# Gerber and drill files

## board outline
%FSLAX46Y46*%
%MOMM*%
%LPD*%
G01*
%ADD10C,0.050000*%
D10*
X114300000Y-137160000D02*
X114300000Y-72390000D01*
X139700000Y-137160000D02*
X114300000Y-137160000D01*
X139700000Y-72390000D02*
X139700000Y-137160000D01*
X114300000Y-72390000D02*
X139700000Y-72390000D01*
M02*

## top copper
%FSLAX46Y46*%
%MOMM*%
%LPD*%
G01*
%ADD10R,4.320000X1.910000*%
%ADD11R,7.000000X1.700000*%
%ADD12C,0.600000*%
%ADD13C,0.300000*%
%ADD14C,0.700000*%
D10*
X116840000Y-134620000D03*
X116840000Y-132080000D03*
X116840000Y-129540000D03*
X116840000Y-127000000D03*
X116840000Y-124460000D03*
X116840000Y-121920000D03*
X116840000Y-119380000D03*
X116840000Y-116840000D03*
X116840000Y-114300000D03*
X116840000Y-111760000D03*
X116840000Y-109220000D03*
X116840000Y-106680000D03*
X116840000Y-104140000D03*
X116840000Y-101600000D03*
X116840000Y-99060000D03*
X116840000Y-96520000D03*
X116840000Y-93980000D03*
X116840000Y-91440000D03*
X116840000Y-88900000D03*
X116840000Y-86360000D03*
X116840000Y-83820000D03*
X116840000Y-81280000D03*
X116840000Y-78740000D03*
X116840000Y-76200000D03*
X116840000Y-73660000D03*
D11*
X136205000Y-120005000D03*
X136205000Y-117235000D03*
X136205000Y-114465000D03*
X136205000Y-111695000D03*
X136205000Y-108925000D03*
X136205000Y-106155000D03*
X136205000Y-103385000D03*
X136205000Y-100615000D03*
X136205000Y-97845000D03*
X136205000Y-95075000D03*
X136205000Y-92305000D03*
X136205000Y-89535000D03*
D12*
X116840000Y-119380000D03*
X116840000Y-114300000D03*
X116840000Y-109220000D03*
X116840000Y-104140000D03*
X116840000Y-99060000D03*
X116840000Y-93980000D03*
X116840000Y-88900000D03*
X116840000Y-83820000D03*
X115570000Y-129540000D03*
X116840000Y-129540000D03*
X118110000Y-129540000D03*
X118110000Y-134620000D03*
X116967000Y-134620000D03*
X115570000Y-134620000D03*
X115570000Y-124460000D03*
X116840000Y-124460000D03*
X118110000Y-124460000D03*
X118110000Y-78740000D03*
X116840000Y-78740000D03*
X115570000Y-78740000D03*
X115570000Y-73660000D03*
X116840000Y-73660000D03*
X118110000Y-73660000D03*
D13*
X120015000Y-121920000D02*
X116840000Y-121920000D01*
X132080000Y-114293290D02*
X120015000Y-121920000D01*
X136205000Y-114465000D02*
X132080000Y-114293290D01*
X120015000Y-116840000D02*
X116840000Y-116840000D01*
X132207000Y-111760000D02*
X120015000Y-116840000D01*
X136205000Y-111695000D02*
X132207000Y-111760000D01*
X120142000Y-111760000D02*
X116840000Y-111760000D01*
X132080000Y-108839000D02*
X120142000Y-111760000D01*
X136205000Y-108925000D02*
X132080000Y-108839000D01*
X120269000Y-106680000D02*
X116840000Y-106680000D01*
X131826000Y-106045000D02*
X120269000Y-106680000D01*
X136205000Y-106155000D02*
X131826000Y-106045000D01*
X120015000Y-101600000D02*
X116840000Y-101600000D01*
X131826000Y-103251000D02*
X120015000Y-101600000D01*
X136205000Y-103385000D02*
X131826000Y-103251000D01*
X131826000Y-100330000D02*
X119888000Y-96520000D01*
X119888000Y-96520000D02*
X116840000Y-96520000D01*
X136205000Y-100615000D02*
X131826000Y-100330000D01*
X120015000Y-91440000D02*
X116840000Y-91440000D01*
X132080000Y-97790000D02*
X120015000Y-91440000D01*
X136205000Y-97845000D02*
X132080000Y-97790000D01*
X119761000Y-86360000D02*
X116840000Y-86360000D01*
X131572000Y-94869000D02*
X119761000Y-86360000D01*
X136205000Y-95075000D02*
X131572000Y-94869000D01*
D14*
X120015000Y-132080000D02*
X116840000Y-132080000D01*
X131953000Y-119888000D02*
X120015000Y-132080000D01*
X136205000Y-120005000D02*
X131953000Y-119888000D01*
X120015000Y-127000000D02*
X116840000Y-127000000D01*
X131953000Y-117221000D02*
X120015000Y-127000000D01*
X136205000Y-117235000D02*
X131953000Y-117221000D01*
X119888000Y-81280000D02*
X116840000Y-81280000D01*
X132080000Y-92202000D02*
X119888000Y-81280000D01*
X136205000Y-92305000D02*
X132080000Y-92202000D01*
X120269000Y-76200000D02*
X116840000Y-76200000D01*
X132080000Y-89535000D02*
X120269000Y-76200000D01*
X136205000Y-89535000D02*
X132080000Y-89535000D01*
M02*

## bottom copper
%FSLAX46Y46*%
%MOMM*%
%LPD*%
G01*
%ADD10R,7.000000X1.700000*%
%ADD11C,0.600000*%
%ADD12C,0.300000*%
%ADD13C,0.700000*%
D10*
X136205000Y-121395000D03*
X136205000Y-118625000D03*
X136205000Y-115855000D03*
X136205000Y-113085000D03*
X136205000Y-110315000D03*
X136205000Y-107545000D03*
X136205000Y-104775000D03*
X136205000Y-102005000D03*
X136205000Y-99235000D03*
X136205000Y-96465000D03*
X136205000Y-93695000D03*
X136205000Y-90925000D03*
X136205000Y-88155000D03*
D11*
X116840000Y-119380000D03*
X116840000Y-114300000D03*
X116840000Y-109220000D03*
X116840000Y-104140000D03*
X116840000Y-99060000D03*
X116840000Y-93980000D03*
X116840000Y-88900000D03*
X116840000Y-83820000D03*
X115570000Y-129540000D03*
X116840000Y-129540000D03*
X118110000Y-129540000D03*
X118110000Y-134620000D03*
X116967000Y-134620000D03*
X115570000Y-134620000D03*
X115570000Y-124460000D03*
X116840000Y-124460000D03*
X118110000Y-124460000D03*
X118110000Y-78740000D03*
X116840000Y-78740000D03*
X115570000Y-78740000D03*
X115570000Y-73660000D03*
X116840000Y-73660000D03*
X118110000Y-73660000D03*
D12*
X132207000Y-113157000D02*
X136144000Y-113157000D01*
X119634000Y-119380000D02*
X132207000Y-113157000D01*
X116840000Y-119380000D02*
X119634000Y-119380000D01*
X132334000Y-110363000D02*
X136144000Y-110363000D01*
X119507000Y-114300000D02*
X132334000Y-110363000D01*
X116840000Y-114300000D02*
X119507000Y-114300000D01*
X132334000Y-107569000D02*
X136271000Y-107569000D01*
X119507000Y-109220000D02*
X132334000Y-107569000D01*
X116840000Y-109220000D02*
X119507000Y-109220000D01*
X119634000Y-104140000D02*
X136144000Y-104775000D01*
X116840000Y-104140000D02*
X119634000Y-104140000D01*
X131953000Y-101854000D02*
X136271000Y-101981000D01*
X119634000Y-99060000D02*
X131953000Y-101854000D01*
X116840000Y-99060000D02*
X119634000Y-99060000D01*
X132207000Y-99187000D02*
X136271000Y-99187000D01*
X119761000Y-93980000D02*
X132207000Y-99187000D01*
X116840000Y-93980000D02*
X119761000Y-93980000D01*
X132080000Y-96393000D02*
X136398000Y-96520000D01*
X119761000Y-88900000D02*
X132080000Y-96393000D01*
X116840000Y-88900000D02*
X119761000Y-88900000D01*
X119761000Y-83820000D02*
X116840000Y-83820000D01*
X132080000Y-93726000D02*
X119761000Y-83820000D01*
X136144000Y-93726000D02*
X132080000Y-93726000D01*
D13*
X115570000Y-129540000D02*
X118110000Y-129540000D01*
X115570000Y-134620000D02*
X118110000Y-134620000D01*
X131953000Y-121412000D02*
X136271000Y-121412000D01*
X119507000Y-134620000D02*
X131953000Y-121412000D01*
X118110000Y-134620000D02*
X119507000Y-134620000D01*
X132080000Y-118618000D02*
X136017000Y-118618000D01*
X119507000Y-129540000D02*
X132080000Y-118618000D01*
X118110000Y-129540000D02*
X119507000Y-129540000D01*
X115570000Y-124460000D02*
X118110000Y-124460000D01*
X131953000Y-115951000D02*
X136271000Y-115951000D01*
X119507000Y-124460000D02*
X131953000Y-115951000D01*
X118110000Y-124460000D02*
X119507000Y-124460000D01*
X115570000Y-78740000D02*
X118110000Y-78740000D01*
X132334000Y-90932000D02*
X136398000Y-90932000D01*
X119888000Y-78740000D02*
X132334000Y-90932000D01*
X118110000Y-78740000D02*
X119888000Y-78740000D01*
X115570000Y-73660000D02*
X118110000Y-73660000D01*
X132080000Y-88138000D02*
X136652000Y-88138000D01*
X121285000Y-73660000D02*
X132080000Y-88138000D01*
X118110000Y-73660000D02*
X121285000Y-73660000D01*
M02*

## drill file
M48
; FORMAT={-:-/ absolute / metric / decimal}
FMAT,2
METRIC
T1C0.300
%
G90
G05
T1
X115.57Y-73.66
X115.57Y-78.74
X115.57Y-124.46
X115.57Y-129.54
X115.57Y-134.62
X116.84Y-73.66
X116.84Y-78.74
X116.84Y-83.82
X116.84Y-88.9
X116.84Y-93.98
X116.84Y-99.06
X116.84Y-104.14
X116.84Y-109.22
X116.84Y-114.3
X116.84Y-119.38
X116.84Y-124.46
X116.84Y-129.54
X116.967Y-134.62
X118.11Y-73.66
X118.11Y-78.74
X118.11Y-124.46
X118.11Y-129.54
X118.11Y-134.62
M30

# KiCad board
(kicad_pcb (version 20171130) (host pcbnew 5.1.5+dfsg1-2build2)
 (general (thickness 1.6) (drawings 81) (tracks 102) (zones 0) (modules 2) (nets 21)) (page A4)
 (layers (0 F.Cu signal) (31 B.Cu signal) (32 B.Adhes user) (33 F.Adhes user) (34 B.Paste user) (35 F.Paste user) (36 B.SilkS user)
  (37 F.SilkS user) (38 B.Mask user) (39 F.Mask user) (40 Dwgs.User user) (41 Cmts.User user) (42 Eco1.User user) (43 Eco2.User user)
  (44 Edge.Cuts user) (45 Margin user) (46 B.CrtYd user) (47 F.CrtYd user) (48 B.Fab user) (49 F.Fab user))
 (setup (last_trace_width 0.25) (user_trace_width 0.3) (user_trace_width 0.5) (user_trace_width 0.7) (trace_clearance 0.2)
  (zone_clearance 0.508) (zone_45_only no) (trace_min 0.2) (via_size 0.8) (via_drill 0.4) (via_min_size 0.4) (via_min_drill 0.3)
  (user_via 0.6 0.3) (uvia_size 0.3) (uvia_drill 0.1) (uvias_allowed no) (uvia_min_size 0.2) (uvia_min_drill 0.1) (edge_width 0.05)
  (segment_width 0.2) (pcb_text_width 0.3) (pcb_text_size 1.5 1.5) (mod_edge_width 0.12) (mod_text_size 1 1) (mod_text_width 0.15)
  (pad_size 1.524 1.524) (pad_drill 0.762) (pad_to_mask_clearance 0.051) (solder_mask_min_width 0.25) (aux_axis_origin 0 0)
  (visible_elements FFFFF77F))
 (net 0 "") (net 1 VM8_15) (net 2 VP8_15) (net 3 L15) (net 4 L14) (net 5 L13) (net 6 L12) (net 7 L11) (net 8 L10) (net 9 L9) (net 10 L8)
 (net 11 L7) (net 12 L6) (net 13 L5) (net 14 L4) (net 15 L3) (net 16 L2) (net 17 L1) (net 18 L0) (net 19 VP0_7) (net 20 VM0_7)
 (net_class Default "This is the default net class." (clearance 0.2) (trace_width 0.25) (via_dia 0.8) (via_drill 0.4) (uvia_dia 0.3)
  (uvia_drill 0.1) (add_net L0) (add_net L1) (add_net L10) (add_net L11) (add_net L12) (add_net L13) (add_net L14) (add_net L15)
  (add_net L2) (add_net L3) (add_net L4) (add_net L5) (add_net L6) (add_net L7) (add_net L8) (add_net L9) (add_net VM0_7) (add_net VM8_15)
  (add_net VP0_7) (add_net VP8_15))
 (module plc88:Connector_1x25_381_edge (layer F.Cu) (at 111.76 71.12)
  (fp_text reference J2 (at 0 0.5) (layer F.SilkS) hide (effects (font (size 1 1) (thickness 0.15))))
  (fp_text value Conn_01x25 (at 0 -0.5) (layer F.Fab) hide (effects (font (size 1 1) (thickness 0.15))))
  (pad 25 smd rect (at 5.08 63.5) (size 4.32 1.91) (layers F.Cu F.Paste F.Mask) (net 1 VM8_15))
  (pad 24 smd rect (at 5.08 60.96) (size 4.32 1.91) (layers F.Cu F.Paste F.Mask) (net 1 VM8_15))
  (pad 23 smd rect (at 5.08 58.42) (size 4.32 1.91) (layers F.Cu F.Paste F.Mask) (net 1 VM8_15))
  (pad 22 smd rect (at 5.08 55.88) (size 4.32 1.91) (layers F.Cu F.Paste F.Mask) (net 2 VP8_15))
  (pad 21 smd rect (at 5.08 53.34) (size 4.32 1.91) (layers F.Cu F.Paste F.Mask) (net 2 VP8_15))
  (pad 20 smd rect (at 5.08 50.8) (size 4.32 1.91) (layers F.Cu F.Paste F.Mask) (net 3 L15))
  (pad 19 smd rect (at 5.08 48.26) (size 4.32 1.91) (layers F.Cu F.Paste F.Mask) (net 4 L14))
  (pad 18 smd rect (at 5.08 45.72) (size 4.32 1.91) (layers F.Cu F.Paste F.Mask) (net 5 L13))
  (pad 17 smd rect (at 5.08 43.18) (size 4.32 1.91) (layers F.Cu F.Paste F.Mask) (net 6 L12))
  (pad 16 smd rect (at 5.08 40.64) (size 4.32 1.91) (layers F.Cu F.Paste F.Mask) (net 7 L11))
  (pad 15 smd rect (at 5.08 38.1) (size 4.32 1.91) (layers F.Cu F.Paste F.Mask) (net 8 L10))
  (pad 14 smd rect (at 5.08 35.56) (size 4.32 1.91) (layers F.Cu F.Paste F.Mask) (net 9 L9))
  (pad 13 smd rect (at 5.08 33.02) (size 4.32 1.91) (layers F.Cu F.Paste F.Mask) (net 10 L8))
  (pad 12 smd rect (at 5.08 30.48) (size 4.32 1.91) (layers F.Cu F.Paste F.Mask) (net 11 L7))
  (pad 11 smd rect (at 5.08 27.94) (size 4.32 1.91) (layers F.Cu F.Paste F.Mask) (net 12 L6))
  (pad 10 smd rect (at 5.08 25.4) (size 4.32 1.91) (layers F.Cu F.Paste F.Mask) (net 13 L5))
  (pad 9 smd rect (at 5.08 22.86) (size 4.32 1.91) (layers F.Cu F.Paste F.Mask) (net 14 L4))
  (pad 8 smd rect (at 5.08 20.32) (size 4.32 1.91) (layers F.Cu F.Paste F.Mask) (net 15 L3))
  (pad 7 smd rect (at 5.08 17.78) (size 4.32 1.91) (layers F.Cu F.Paste F.Mask) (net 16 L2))
  (pad 6 smd rect (at 5.08 15.24) (size 4.32 1.91) (layers F.Cu F.Paste F.Mask) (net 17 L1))
  (pad 5 smd rect (at 5.08 12.7) (size 4.32 1.91) (layers F.Cu F.Paste F.Mask) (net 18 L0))
  (pad 4 smd rect (at 5.08 10.16) (size 4.32 1.91) (layers F.Cu F.Paste F.Mask) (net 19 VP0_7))
  (pad 3 smd rect (at 5.08 7.62) (size 4.32 1.91) (layers F.Cu F.Paste F.Mask) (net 19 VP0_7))
  (pad 2 smd rect (at 5.08 5.08) (size 4.32 1.91) (layers F.Cu F.Paste F.Mask) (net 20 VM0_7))
  (pad 1 smd rect (at 5.08 2.54) (size 4.32 1.91) (layers F.Cu F.Paste F.Mask) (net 20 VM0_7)))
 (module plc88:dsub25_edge (layer F.Cu) (at 132.715 85.665)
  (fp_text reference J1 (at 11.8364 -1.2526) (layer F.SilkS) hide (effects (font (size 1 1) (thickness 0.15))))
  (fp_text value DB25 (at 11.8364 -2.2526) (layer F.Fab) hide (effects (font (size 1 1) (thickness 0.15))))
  (pad 25 smd rect (at 3.49 34.34) (size 7 1.7) (layers F.Cu F.Paste F.Mask) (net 1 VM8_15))
  (pad 24 smd rect (at 3.49 31.57) (size 7 1.7) (layers F.Cu F.Paste F.Mask) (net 2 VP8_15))
  (pad 23 smd rect (at 3.49 28.8) (size 7 1.7) (layers F.Cu F.Paste F.Mask) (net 3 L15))
  (pad 22 smd rect (at 3.49 26.03) (size 7 1.7) (layers F.Cu F.Paste F.Mask) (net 5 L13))
  (pad 21 smd rect (at 3.49 23.26) (size 7 1.7) (layers F.Cu F.Paste F.Mask) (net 7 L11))
  (pad 20 smd rect (at 3.49 20.49) (size 7 1.7) (layers F.Cu F.Paste F.Mask) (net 9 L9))
  (pad 19 smd rect (at 3.49 17.72) (size 7 1.7) (layers F.Cu F.Paste F.Mask) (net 11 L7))
  (pad 18 smd rect (at 3.49 14.95) (size 7 1.7) (layers F.Cu F.Paste F.Mask) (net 13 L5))
  (pad 17 smd rect (at 3.49 12.18) (size 7 1.7) (layers F.Cu F.Paste F.Mask) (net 15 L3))
  (pad 16 smd rect (at 3.49 9.41) (size 7 1.7) (layers F.Cu F.Paste F.Mask) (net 17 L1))
  (pad 15 smd rect (at 3.49 6.64) (size 7 1.7) (layers F.Cu F.Paste F.Mask) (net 19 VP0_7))
  (pad 14 smd rect (at 3.49 3.87) (size 7 1.7) (layers F.Cu F.Paste F.Mask) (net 20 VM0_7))
  (pad 13 smd rect (at 3.49 35.73) (size 7 1.7) (layers B.Cu B.Paste B.Mask) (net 1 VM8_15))
  (pad 12 smd rect (at 3.49 32.96) (size 7 1.7) (layers B.Cu B.Paste B.Mask) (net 1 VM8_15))
  (pad 11 smd rect (at 3.49 30.19) (size 7 1.7) (layers B.Cu B.Paste B.Mask) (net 2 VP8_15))
  (pad 10 smd rect (at 3.49 27.42) (size 7 1.7) (layers B.Cu B.Paste B.Mask) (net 4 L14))
  (pad 9 smd rect (at 3.49 24.65) (size 7 1.7) (layers B.Cu B.Paste B.Mask) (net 6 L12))
  (pad 8 smd rect (at 3.49 21.88) (size 7 1.7) (layers B.Cu B.Paste B.Mask) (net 8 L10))
  (pad 7 smd rect (at 3.49 19.11) (size 7 1.7) (layers B.Cu B.Paste B.Mask) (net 10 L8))
  (pad 6 smd rect (at 3.49 16.34) (size 7 1.7) (layers B.Cu B.Paste B.Mask) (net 12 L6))
  (pad 5 smd rect (at 3.49 13.57) (size 7 1.7) (layers B.Cu B.Paste B.Mask) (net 14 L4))
  (pad 4 smd rect (at 3.49 10.8) (size 7 1.7) (layers B.Cu B.Paste B.Mask) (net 16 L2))
  (pad 3 smd rect (at 3.49 8.03) (size 7 1.7) (layers B.Cu B.Paste B.Mask) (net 18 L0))
  (pad 2 smd rect (at 3.49 5.26) (size 7 1.7) (layers B.Cu B.Paste B.Mask) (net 19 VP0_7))
  (pad 1 smd rect (at 3.49 2.49) (size 7 1.7) (layers B.Cu B.Paste B.Mask) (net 20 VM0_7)))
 (gr_line (start 114.3 137.16) (end 114.3 72.39) (layer Edge.Cuts) (width 0.05))
 (gr_line (start 139.7 137.16) (end 114.3 137.16) (layer Edge.Cuts) (width 0.05))
 (gr_line (start 139.7 72.39) (end 139.7 137.16) (layer Edge.Cuts) (width 0.05))
 (gr_line (start 114.3 72.39) (end 139.7 72.39) (layer Edge.Cuts) (width 0.05))
 (segment (start 120.015 121.92) (end 116.84 121.92) (width 0.3) (layer F.Cu) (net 3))
 (segment (start 132.08 114.29329) (end 120.015 121.92) (width 0.3) (layer F.Cu) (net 3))
 (segment (start 136.205 114.465) (end 132.08 114.29329) (width 0.3) (layer F.Cu) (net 3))
 (segment (start 120.015 116.84) (end 116.84 116.84) (width 0.3) (layer F.Cu) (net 5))
 (segment (start 132.207 111.76) (end 120.015 116.84) (width 0.3) (layer F.Cu) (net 5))
 (segment (start 136.205 111.695) (end 132.207 111.76) (width 0.3) (layer F.Cu) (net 5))
 (segment (start 120.142 111.76) (end 116.84 111.76) (width 0.3) (layer F.Cu) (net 7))
 (segment (start 132.08 108.839) (end 120.142 111.76) (width 0.3) (layer F.Cu) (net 7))
 (segment (start 136.205 108.925) (end 132.08 108.839) (width 0.3) (layer F.Cu) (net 7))
 (segment (start 120.269 106.68) (end 116.84 106.68) (width 0.3) (layer F.Cu) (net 9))
 (segment (start 131.826 106.045) (end 120.269 106.68) (width 0.3) (layer F.Cu) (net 9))
 (segment (start 136.205 106.155) (end 131.826 106.045) (width 0.3) (layer F.Cu) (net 9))
 (segment (start 120.015 101.6) (end 116.84 101.6) (width 0.3) (layer F.Cu) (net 11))
 (segment (start 131.826 103.251) (end 120.015 101.6) (width 0.3) (layer F.Cu) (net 11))
 (segment (start 136.205 103.385) (end 131.826 103.251) (width 0.3) (layer F.Cu) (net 11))
 (segment (start 131.826 100.33) (end 119.888 96.52) (width 0.3) (layer F.Cu) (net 13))
 (segment (start 119.888 96.52) (end 116.84 96.52) (width 0.3) (layer F.Cu) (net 13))
 (segment (start 136.205 100.615) (end 131.826 100.33) (width 0.3) (layer F.Cu) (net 13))
 (segment (start 120.015 91.44) (end 116.84 91.44) (width 0.3) (layer F.Cu) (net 15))
 (segment (start 132.08 97.79) (end 120.015 91.44) (width 0.3) (layer F.Cu) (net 15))
 (segment (start 136.205 97.845) (end 132.08 97.79) (width 0.3) (layer F.Cu) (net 15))
 (segment (start 119.761 86.36) (end 116.84 86.36) (width 0.3) (layer F.Cu) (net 17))
 (segment (start 131.572 94.869) (end 119.761 86.36) (width 0.3) (layer F.Cu) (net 17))
 (segment (start 136.205 95.075) (end 131.572 94.869) (width 0.3) (layer F.Cu) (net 17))
 (via (at 116.84 119.38) (size 0.6) (drill 0.3) (layers F.Cu B.Cu) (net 4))
 (segment (start 132.207 113.157) (end 136.144 113.157) (width 0.3) (layer B.Cu) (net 4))
 (segment (start 119.634 119.38) (end 132.207 113.157) (width 0.3) (layer B.Cu) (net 4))
 (segment (start 116.84 119.38) (end 119.634 119.38) (width 0.3) (layer B.Cu) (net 4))
 (via (at 116.84 114.3) (size 0.6) (drill 0.3) (layers F.Cu B.Cu) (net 6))
 (segment (start 132.334 110.363) (end 136.144 110.363) (width 0.3) (layer B.Cu) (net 6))
 (segment (start 119.507 114.3) (end 132.334 110.363) (width 0.3) (layer B.Cu) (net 6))
 (segment (start 116.84 114.3) (end 119.507 114.3) (width 0.3) (layer B.Cu) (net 6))
 (via (at 116.84 109.22) (size 0.6) (drill 0.3) (layers F.Cu B.Cu) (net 8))
 (segment (start 132.334 107.569) (end 136.271 107.569) (width 0.3) (layer B.Cu) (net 8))
 (segment (start 119.507 109.22) (end 132.334 107.569) (width 0.3) (layer B.Cu) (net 8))
 (segment (start 116.84 109.22) (end 119.507 109.22) (width 0.3) (layer B.Cu) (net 8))
 (via (at 116.84 104.14) (size 0.6) (drill 0.3) (layers F.Cu B.Cu) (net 10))
 (segment (start 119.634 104.14) (end 136.144 104.775) (width 0.3) (layer B.Cu) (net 10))
 (segment (start 116.84 104.14) (end 119.634 104.14) (width 0.3) (layer B.Cu) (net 10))
 (via (at 116.84 99.06) (size 0.6) (drill 0.3) (layers F.Cu B.Cu) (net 12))
 (segment (start 131.953 101.854) (end 136.271 101.981) (width 0.3) (layer B.Cu) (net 12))
 (segment (start 119.634 99.06) (end 131.953 101.854) (width 0.3) (layer B.Cu) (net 12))
 (segment (start 116.84 99.06) (end 119.634 99.06) (width 0.3) (layer B.Cu) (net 12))
 (via (at 116.84 93.98) (size 0.6) (drill 0.3) (layers F.Cu B.Cu) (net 14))
 (segment (start 132.207 99.187) (end 136.271 99.187) (width 0.3) (layer B.Cu) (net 14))
 (segment (start 119.761 93.98) (end 132.207 99.187) (width 0.3) (layer B.Cu) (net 14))
 (segment (start 116.84 93.98) (end 119.761 93.98) (width 0.3) (layer B.Cu) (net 14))
 (via (at 116.84 88.9) (size 0.6) (drill 0.3) (layers F.Cu B.Cu) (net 16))
 (segment (start 132.08 96.393) (end 136.398 96.52) (width 0.3) (layer B.Cu) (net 16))
 (segment (start 119.761 88.9) (end 132.08 96.393) (width 0.3) (layer B.Cu) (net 16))
 (segment (start 116.84 88.9) (end 119.761 88.9) (width 0.3) (layer B.Cu) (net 16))
 (via (at 116.84 83.82) (size 0.6) (drill 0.3) (layers F.Cu B.Cu) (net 18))
 (segment (start 119.761 83.82) (end 116.84 83.82) (width 0.3) (layer B.Cu) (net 18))
 (segment (start 132.08 93.726) (end 119.761 83.82) (width 0.3) (layer B.Cu) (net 18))
 (segment (start 136.144 93.726) (end 132.08 93.726) (width 0.3) (layer B.Cu) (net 18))
 (via (at 115.57 129.54) (size 0.6) (drill 0.3) (layers F.Cu B.Cu) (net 1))
 (via (at 116.84 129.54) (size 0.6) (drill 0.3) (layers F.Cu B.Cu) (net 1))
 (via (at 118.11 129.54) (size 0.6) (drill 0.3) (layers F.Cu B.Cu) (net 1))
 (via (at 118.11 134.62) (size 0.6) (drill 0.3) (layers F.Cu B.Cu) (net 1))
 (via (at 116.967 134.62) (size 0.6) (drill 0.3) (layers F.Cu B.Cu) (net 1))
 (via (at 115.57 134.62) (size 0.6) (drill 0.3) (layers F.Cu B.Cu) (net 1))
 (segment (start 115.57 129.54) (end 118.11 129.54) (width 0.7) (layer B.Cu) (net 1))
 (segment (start 115.57 134.62) (end 118.11 134.62) (width 0.7) (layer B.Cu) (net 1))
 (segment (start 120.015 132.08) (end 116.84 132.08) (width 0.7) (layer F.Cu) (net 1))
 (segment (start 131.953 119.888) (end 120.015 132.08) (width 0.7) (layer F.Cu) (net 1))
 (segment (start 136.205 120.005) (end 131.953 119.888) (width 0.7) (layer F.Cu) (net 1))
 (segment (start 131.953 121.412) (end 136.271 121.412) (width 0.7) (layer B.Cu) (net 1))
 (segment (start 119.507 134.62) (end 131.953 121.412) (width 0.7) (layer B.Cu) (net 1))
 (segment (start 118.11 134.62) (end 119.507 134.62) (width 0.7) (layer B.Cu) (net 1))
 (segment (start 132.08 118.618) (end 136.017 118.618) (width 0.7) (layer B.Cu) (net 1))
 (segment (start 119.507 129.54) (end 132.08 118.618) (width 0.7) (layer B.Cu) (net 1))
 (segment (start 118.11 129.54) (end 119.507 129.54) (width 0.7) (layer B.Cu) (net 1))
 (via (at 115.57 124.46) (size 0.6) (drill 0.3) (layers F.Cu B.Cu) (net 2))
 (via (at 116.84 124.46) (size 0.6) (drill 0.3) (layers F.Cu B.Cu) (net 2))
 (via (at 118.11 124.46) (size 0.6) (drill 0.3) (layers F.Cu B.Cu) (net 2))
 (segment (start 115.57 124.46) (end 118.11 124.46) (width 0.7) (layer B.Cu) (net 2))
 (segment (start 120.015 127) (end 116.84 127) (width 0.7) (layer F.Cu) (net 2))
 (segment (start 131.953 117.221) (end 120.015 127) (width 0.7) (layer F.Cu) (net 2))
 (segment (start 136.205 117.235) (end 131.953 117.221) (width 0.7) (layer F.Cu) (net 2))
 (segment (start 131.953 115.951) (end 136.271 115.951) (width 0.7) (layer B.Cu) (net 2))
 (segment (start 119.507 124.46) (end 131.953 115.951) (width 0.7) (layer B.Cu) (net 2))
 (segment (start 118.11 124.46) (end 119.507 124.46) (width 0.7) (layer B.Cu) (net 2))
 (via (at 118.11 78.74) (size 0.6) (drill 0.3) (layers F.Cu B.Cu) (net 19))
 (via (at 116.84 78.74) (size 0.6) (drill 0.3) (layers F.Cu B.Cu) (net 19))
 (via (at 115.57 78.74) (size 0.6) (drill 0.3) (layers F.Cu B.Cu) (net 19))
 (segment (start 115.57 78.74) (end 118.11 78.74) (width 0.7) (layer B.Cu) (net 19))
 (segment (start 119.888 81.28) (end 116.84 81.28) (width 0.7) (layer F.Cu) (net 19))
 (segment (start 132.08 92.202) (end 119.888 81.28) (width 0.7) (layer F.Cu) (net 19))
 (segment (start 136.205 92.305) (end 132.08 92.202) (width 0.7) (layer F.Cu) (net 19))
 (segment (start 132.334 90.932) (end 136.398 90.932) (width 0.7) (layer B.Cu) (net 19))
 (segment (start 119.888 78.74) (end 132.334 90.932) (width 0.7) (layer B.Cu) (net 19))
 (segment (start 118.11 78.74) (end 119.888 78.74) (width 0.7) (layer B.Cu) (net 19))
 (via (at 115.57 73.66) (size 0.6) (drill 0.3) (layers F.Cu B.Cu) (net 20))
 (via (at 116.84 73.66) (size 0.6) (drill 0.3) (layers F.Cu B.Cu) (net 20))
 (via (at 118.11 73.66) (size 0.6) (drill 0.3) (layers F.Cu B.Cu) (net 20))
 (segment (start 115.57 73.66) (end 118.11 73.66) (width 0.7) (layer B.Cu) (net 20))
 (segment (start 120.269 76.2) (end 116.84 76.2) (width 0.7) (layer F.Cu) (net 20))
 (segment (start 132.08 89.535) (end 120.269 76.2) (width 0.7) (layer F.Cu) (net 20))
 (segment (start 136.205 89.535) (end 132.08 89.535) (width 0.7) (layer F.Cu) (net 20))
 (segment (start 132.08 88.138) (end 136.652 88.138) (width 0.7) (layer B.Cu) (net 20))
 (segment (start 121.285 73.66) (end 132.08 88.138) (width 0.7) (layer B.Cu) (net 20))
 (segment (start 118.11 73.66) (end 121.285 73.66) (width 0.7) (layer B.Cu) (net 20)))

